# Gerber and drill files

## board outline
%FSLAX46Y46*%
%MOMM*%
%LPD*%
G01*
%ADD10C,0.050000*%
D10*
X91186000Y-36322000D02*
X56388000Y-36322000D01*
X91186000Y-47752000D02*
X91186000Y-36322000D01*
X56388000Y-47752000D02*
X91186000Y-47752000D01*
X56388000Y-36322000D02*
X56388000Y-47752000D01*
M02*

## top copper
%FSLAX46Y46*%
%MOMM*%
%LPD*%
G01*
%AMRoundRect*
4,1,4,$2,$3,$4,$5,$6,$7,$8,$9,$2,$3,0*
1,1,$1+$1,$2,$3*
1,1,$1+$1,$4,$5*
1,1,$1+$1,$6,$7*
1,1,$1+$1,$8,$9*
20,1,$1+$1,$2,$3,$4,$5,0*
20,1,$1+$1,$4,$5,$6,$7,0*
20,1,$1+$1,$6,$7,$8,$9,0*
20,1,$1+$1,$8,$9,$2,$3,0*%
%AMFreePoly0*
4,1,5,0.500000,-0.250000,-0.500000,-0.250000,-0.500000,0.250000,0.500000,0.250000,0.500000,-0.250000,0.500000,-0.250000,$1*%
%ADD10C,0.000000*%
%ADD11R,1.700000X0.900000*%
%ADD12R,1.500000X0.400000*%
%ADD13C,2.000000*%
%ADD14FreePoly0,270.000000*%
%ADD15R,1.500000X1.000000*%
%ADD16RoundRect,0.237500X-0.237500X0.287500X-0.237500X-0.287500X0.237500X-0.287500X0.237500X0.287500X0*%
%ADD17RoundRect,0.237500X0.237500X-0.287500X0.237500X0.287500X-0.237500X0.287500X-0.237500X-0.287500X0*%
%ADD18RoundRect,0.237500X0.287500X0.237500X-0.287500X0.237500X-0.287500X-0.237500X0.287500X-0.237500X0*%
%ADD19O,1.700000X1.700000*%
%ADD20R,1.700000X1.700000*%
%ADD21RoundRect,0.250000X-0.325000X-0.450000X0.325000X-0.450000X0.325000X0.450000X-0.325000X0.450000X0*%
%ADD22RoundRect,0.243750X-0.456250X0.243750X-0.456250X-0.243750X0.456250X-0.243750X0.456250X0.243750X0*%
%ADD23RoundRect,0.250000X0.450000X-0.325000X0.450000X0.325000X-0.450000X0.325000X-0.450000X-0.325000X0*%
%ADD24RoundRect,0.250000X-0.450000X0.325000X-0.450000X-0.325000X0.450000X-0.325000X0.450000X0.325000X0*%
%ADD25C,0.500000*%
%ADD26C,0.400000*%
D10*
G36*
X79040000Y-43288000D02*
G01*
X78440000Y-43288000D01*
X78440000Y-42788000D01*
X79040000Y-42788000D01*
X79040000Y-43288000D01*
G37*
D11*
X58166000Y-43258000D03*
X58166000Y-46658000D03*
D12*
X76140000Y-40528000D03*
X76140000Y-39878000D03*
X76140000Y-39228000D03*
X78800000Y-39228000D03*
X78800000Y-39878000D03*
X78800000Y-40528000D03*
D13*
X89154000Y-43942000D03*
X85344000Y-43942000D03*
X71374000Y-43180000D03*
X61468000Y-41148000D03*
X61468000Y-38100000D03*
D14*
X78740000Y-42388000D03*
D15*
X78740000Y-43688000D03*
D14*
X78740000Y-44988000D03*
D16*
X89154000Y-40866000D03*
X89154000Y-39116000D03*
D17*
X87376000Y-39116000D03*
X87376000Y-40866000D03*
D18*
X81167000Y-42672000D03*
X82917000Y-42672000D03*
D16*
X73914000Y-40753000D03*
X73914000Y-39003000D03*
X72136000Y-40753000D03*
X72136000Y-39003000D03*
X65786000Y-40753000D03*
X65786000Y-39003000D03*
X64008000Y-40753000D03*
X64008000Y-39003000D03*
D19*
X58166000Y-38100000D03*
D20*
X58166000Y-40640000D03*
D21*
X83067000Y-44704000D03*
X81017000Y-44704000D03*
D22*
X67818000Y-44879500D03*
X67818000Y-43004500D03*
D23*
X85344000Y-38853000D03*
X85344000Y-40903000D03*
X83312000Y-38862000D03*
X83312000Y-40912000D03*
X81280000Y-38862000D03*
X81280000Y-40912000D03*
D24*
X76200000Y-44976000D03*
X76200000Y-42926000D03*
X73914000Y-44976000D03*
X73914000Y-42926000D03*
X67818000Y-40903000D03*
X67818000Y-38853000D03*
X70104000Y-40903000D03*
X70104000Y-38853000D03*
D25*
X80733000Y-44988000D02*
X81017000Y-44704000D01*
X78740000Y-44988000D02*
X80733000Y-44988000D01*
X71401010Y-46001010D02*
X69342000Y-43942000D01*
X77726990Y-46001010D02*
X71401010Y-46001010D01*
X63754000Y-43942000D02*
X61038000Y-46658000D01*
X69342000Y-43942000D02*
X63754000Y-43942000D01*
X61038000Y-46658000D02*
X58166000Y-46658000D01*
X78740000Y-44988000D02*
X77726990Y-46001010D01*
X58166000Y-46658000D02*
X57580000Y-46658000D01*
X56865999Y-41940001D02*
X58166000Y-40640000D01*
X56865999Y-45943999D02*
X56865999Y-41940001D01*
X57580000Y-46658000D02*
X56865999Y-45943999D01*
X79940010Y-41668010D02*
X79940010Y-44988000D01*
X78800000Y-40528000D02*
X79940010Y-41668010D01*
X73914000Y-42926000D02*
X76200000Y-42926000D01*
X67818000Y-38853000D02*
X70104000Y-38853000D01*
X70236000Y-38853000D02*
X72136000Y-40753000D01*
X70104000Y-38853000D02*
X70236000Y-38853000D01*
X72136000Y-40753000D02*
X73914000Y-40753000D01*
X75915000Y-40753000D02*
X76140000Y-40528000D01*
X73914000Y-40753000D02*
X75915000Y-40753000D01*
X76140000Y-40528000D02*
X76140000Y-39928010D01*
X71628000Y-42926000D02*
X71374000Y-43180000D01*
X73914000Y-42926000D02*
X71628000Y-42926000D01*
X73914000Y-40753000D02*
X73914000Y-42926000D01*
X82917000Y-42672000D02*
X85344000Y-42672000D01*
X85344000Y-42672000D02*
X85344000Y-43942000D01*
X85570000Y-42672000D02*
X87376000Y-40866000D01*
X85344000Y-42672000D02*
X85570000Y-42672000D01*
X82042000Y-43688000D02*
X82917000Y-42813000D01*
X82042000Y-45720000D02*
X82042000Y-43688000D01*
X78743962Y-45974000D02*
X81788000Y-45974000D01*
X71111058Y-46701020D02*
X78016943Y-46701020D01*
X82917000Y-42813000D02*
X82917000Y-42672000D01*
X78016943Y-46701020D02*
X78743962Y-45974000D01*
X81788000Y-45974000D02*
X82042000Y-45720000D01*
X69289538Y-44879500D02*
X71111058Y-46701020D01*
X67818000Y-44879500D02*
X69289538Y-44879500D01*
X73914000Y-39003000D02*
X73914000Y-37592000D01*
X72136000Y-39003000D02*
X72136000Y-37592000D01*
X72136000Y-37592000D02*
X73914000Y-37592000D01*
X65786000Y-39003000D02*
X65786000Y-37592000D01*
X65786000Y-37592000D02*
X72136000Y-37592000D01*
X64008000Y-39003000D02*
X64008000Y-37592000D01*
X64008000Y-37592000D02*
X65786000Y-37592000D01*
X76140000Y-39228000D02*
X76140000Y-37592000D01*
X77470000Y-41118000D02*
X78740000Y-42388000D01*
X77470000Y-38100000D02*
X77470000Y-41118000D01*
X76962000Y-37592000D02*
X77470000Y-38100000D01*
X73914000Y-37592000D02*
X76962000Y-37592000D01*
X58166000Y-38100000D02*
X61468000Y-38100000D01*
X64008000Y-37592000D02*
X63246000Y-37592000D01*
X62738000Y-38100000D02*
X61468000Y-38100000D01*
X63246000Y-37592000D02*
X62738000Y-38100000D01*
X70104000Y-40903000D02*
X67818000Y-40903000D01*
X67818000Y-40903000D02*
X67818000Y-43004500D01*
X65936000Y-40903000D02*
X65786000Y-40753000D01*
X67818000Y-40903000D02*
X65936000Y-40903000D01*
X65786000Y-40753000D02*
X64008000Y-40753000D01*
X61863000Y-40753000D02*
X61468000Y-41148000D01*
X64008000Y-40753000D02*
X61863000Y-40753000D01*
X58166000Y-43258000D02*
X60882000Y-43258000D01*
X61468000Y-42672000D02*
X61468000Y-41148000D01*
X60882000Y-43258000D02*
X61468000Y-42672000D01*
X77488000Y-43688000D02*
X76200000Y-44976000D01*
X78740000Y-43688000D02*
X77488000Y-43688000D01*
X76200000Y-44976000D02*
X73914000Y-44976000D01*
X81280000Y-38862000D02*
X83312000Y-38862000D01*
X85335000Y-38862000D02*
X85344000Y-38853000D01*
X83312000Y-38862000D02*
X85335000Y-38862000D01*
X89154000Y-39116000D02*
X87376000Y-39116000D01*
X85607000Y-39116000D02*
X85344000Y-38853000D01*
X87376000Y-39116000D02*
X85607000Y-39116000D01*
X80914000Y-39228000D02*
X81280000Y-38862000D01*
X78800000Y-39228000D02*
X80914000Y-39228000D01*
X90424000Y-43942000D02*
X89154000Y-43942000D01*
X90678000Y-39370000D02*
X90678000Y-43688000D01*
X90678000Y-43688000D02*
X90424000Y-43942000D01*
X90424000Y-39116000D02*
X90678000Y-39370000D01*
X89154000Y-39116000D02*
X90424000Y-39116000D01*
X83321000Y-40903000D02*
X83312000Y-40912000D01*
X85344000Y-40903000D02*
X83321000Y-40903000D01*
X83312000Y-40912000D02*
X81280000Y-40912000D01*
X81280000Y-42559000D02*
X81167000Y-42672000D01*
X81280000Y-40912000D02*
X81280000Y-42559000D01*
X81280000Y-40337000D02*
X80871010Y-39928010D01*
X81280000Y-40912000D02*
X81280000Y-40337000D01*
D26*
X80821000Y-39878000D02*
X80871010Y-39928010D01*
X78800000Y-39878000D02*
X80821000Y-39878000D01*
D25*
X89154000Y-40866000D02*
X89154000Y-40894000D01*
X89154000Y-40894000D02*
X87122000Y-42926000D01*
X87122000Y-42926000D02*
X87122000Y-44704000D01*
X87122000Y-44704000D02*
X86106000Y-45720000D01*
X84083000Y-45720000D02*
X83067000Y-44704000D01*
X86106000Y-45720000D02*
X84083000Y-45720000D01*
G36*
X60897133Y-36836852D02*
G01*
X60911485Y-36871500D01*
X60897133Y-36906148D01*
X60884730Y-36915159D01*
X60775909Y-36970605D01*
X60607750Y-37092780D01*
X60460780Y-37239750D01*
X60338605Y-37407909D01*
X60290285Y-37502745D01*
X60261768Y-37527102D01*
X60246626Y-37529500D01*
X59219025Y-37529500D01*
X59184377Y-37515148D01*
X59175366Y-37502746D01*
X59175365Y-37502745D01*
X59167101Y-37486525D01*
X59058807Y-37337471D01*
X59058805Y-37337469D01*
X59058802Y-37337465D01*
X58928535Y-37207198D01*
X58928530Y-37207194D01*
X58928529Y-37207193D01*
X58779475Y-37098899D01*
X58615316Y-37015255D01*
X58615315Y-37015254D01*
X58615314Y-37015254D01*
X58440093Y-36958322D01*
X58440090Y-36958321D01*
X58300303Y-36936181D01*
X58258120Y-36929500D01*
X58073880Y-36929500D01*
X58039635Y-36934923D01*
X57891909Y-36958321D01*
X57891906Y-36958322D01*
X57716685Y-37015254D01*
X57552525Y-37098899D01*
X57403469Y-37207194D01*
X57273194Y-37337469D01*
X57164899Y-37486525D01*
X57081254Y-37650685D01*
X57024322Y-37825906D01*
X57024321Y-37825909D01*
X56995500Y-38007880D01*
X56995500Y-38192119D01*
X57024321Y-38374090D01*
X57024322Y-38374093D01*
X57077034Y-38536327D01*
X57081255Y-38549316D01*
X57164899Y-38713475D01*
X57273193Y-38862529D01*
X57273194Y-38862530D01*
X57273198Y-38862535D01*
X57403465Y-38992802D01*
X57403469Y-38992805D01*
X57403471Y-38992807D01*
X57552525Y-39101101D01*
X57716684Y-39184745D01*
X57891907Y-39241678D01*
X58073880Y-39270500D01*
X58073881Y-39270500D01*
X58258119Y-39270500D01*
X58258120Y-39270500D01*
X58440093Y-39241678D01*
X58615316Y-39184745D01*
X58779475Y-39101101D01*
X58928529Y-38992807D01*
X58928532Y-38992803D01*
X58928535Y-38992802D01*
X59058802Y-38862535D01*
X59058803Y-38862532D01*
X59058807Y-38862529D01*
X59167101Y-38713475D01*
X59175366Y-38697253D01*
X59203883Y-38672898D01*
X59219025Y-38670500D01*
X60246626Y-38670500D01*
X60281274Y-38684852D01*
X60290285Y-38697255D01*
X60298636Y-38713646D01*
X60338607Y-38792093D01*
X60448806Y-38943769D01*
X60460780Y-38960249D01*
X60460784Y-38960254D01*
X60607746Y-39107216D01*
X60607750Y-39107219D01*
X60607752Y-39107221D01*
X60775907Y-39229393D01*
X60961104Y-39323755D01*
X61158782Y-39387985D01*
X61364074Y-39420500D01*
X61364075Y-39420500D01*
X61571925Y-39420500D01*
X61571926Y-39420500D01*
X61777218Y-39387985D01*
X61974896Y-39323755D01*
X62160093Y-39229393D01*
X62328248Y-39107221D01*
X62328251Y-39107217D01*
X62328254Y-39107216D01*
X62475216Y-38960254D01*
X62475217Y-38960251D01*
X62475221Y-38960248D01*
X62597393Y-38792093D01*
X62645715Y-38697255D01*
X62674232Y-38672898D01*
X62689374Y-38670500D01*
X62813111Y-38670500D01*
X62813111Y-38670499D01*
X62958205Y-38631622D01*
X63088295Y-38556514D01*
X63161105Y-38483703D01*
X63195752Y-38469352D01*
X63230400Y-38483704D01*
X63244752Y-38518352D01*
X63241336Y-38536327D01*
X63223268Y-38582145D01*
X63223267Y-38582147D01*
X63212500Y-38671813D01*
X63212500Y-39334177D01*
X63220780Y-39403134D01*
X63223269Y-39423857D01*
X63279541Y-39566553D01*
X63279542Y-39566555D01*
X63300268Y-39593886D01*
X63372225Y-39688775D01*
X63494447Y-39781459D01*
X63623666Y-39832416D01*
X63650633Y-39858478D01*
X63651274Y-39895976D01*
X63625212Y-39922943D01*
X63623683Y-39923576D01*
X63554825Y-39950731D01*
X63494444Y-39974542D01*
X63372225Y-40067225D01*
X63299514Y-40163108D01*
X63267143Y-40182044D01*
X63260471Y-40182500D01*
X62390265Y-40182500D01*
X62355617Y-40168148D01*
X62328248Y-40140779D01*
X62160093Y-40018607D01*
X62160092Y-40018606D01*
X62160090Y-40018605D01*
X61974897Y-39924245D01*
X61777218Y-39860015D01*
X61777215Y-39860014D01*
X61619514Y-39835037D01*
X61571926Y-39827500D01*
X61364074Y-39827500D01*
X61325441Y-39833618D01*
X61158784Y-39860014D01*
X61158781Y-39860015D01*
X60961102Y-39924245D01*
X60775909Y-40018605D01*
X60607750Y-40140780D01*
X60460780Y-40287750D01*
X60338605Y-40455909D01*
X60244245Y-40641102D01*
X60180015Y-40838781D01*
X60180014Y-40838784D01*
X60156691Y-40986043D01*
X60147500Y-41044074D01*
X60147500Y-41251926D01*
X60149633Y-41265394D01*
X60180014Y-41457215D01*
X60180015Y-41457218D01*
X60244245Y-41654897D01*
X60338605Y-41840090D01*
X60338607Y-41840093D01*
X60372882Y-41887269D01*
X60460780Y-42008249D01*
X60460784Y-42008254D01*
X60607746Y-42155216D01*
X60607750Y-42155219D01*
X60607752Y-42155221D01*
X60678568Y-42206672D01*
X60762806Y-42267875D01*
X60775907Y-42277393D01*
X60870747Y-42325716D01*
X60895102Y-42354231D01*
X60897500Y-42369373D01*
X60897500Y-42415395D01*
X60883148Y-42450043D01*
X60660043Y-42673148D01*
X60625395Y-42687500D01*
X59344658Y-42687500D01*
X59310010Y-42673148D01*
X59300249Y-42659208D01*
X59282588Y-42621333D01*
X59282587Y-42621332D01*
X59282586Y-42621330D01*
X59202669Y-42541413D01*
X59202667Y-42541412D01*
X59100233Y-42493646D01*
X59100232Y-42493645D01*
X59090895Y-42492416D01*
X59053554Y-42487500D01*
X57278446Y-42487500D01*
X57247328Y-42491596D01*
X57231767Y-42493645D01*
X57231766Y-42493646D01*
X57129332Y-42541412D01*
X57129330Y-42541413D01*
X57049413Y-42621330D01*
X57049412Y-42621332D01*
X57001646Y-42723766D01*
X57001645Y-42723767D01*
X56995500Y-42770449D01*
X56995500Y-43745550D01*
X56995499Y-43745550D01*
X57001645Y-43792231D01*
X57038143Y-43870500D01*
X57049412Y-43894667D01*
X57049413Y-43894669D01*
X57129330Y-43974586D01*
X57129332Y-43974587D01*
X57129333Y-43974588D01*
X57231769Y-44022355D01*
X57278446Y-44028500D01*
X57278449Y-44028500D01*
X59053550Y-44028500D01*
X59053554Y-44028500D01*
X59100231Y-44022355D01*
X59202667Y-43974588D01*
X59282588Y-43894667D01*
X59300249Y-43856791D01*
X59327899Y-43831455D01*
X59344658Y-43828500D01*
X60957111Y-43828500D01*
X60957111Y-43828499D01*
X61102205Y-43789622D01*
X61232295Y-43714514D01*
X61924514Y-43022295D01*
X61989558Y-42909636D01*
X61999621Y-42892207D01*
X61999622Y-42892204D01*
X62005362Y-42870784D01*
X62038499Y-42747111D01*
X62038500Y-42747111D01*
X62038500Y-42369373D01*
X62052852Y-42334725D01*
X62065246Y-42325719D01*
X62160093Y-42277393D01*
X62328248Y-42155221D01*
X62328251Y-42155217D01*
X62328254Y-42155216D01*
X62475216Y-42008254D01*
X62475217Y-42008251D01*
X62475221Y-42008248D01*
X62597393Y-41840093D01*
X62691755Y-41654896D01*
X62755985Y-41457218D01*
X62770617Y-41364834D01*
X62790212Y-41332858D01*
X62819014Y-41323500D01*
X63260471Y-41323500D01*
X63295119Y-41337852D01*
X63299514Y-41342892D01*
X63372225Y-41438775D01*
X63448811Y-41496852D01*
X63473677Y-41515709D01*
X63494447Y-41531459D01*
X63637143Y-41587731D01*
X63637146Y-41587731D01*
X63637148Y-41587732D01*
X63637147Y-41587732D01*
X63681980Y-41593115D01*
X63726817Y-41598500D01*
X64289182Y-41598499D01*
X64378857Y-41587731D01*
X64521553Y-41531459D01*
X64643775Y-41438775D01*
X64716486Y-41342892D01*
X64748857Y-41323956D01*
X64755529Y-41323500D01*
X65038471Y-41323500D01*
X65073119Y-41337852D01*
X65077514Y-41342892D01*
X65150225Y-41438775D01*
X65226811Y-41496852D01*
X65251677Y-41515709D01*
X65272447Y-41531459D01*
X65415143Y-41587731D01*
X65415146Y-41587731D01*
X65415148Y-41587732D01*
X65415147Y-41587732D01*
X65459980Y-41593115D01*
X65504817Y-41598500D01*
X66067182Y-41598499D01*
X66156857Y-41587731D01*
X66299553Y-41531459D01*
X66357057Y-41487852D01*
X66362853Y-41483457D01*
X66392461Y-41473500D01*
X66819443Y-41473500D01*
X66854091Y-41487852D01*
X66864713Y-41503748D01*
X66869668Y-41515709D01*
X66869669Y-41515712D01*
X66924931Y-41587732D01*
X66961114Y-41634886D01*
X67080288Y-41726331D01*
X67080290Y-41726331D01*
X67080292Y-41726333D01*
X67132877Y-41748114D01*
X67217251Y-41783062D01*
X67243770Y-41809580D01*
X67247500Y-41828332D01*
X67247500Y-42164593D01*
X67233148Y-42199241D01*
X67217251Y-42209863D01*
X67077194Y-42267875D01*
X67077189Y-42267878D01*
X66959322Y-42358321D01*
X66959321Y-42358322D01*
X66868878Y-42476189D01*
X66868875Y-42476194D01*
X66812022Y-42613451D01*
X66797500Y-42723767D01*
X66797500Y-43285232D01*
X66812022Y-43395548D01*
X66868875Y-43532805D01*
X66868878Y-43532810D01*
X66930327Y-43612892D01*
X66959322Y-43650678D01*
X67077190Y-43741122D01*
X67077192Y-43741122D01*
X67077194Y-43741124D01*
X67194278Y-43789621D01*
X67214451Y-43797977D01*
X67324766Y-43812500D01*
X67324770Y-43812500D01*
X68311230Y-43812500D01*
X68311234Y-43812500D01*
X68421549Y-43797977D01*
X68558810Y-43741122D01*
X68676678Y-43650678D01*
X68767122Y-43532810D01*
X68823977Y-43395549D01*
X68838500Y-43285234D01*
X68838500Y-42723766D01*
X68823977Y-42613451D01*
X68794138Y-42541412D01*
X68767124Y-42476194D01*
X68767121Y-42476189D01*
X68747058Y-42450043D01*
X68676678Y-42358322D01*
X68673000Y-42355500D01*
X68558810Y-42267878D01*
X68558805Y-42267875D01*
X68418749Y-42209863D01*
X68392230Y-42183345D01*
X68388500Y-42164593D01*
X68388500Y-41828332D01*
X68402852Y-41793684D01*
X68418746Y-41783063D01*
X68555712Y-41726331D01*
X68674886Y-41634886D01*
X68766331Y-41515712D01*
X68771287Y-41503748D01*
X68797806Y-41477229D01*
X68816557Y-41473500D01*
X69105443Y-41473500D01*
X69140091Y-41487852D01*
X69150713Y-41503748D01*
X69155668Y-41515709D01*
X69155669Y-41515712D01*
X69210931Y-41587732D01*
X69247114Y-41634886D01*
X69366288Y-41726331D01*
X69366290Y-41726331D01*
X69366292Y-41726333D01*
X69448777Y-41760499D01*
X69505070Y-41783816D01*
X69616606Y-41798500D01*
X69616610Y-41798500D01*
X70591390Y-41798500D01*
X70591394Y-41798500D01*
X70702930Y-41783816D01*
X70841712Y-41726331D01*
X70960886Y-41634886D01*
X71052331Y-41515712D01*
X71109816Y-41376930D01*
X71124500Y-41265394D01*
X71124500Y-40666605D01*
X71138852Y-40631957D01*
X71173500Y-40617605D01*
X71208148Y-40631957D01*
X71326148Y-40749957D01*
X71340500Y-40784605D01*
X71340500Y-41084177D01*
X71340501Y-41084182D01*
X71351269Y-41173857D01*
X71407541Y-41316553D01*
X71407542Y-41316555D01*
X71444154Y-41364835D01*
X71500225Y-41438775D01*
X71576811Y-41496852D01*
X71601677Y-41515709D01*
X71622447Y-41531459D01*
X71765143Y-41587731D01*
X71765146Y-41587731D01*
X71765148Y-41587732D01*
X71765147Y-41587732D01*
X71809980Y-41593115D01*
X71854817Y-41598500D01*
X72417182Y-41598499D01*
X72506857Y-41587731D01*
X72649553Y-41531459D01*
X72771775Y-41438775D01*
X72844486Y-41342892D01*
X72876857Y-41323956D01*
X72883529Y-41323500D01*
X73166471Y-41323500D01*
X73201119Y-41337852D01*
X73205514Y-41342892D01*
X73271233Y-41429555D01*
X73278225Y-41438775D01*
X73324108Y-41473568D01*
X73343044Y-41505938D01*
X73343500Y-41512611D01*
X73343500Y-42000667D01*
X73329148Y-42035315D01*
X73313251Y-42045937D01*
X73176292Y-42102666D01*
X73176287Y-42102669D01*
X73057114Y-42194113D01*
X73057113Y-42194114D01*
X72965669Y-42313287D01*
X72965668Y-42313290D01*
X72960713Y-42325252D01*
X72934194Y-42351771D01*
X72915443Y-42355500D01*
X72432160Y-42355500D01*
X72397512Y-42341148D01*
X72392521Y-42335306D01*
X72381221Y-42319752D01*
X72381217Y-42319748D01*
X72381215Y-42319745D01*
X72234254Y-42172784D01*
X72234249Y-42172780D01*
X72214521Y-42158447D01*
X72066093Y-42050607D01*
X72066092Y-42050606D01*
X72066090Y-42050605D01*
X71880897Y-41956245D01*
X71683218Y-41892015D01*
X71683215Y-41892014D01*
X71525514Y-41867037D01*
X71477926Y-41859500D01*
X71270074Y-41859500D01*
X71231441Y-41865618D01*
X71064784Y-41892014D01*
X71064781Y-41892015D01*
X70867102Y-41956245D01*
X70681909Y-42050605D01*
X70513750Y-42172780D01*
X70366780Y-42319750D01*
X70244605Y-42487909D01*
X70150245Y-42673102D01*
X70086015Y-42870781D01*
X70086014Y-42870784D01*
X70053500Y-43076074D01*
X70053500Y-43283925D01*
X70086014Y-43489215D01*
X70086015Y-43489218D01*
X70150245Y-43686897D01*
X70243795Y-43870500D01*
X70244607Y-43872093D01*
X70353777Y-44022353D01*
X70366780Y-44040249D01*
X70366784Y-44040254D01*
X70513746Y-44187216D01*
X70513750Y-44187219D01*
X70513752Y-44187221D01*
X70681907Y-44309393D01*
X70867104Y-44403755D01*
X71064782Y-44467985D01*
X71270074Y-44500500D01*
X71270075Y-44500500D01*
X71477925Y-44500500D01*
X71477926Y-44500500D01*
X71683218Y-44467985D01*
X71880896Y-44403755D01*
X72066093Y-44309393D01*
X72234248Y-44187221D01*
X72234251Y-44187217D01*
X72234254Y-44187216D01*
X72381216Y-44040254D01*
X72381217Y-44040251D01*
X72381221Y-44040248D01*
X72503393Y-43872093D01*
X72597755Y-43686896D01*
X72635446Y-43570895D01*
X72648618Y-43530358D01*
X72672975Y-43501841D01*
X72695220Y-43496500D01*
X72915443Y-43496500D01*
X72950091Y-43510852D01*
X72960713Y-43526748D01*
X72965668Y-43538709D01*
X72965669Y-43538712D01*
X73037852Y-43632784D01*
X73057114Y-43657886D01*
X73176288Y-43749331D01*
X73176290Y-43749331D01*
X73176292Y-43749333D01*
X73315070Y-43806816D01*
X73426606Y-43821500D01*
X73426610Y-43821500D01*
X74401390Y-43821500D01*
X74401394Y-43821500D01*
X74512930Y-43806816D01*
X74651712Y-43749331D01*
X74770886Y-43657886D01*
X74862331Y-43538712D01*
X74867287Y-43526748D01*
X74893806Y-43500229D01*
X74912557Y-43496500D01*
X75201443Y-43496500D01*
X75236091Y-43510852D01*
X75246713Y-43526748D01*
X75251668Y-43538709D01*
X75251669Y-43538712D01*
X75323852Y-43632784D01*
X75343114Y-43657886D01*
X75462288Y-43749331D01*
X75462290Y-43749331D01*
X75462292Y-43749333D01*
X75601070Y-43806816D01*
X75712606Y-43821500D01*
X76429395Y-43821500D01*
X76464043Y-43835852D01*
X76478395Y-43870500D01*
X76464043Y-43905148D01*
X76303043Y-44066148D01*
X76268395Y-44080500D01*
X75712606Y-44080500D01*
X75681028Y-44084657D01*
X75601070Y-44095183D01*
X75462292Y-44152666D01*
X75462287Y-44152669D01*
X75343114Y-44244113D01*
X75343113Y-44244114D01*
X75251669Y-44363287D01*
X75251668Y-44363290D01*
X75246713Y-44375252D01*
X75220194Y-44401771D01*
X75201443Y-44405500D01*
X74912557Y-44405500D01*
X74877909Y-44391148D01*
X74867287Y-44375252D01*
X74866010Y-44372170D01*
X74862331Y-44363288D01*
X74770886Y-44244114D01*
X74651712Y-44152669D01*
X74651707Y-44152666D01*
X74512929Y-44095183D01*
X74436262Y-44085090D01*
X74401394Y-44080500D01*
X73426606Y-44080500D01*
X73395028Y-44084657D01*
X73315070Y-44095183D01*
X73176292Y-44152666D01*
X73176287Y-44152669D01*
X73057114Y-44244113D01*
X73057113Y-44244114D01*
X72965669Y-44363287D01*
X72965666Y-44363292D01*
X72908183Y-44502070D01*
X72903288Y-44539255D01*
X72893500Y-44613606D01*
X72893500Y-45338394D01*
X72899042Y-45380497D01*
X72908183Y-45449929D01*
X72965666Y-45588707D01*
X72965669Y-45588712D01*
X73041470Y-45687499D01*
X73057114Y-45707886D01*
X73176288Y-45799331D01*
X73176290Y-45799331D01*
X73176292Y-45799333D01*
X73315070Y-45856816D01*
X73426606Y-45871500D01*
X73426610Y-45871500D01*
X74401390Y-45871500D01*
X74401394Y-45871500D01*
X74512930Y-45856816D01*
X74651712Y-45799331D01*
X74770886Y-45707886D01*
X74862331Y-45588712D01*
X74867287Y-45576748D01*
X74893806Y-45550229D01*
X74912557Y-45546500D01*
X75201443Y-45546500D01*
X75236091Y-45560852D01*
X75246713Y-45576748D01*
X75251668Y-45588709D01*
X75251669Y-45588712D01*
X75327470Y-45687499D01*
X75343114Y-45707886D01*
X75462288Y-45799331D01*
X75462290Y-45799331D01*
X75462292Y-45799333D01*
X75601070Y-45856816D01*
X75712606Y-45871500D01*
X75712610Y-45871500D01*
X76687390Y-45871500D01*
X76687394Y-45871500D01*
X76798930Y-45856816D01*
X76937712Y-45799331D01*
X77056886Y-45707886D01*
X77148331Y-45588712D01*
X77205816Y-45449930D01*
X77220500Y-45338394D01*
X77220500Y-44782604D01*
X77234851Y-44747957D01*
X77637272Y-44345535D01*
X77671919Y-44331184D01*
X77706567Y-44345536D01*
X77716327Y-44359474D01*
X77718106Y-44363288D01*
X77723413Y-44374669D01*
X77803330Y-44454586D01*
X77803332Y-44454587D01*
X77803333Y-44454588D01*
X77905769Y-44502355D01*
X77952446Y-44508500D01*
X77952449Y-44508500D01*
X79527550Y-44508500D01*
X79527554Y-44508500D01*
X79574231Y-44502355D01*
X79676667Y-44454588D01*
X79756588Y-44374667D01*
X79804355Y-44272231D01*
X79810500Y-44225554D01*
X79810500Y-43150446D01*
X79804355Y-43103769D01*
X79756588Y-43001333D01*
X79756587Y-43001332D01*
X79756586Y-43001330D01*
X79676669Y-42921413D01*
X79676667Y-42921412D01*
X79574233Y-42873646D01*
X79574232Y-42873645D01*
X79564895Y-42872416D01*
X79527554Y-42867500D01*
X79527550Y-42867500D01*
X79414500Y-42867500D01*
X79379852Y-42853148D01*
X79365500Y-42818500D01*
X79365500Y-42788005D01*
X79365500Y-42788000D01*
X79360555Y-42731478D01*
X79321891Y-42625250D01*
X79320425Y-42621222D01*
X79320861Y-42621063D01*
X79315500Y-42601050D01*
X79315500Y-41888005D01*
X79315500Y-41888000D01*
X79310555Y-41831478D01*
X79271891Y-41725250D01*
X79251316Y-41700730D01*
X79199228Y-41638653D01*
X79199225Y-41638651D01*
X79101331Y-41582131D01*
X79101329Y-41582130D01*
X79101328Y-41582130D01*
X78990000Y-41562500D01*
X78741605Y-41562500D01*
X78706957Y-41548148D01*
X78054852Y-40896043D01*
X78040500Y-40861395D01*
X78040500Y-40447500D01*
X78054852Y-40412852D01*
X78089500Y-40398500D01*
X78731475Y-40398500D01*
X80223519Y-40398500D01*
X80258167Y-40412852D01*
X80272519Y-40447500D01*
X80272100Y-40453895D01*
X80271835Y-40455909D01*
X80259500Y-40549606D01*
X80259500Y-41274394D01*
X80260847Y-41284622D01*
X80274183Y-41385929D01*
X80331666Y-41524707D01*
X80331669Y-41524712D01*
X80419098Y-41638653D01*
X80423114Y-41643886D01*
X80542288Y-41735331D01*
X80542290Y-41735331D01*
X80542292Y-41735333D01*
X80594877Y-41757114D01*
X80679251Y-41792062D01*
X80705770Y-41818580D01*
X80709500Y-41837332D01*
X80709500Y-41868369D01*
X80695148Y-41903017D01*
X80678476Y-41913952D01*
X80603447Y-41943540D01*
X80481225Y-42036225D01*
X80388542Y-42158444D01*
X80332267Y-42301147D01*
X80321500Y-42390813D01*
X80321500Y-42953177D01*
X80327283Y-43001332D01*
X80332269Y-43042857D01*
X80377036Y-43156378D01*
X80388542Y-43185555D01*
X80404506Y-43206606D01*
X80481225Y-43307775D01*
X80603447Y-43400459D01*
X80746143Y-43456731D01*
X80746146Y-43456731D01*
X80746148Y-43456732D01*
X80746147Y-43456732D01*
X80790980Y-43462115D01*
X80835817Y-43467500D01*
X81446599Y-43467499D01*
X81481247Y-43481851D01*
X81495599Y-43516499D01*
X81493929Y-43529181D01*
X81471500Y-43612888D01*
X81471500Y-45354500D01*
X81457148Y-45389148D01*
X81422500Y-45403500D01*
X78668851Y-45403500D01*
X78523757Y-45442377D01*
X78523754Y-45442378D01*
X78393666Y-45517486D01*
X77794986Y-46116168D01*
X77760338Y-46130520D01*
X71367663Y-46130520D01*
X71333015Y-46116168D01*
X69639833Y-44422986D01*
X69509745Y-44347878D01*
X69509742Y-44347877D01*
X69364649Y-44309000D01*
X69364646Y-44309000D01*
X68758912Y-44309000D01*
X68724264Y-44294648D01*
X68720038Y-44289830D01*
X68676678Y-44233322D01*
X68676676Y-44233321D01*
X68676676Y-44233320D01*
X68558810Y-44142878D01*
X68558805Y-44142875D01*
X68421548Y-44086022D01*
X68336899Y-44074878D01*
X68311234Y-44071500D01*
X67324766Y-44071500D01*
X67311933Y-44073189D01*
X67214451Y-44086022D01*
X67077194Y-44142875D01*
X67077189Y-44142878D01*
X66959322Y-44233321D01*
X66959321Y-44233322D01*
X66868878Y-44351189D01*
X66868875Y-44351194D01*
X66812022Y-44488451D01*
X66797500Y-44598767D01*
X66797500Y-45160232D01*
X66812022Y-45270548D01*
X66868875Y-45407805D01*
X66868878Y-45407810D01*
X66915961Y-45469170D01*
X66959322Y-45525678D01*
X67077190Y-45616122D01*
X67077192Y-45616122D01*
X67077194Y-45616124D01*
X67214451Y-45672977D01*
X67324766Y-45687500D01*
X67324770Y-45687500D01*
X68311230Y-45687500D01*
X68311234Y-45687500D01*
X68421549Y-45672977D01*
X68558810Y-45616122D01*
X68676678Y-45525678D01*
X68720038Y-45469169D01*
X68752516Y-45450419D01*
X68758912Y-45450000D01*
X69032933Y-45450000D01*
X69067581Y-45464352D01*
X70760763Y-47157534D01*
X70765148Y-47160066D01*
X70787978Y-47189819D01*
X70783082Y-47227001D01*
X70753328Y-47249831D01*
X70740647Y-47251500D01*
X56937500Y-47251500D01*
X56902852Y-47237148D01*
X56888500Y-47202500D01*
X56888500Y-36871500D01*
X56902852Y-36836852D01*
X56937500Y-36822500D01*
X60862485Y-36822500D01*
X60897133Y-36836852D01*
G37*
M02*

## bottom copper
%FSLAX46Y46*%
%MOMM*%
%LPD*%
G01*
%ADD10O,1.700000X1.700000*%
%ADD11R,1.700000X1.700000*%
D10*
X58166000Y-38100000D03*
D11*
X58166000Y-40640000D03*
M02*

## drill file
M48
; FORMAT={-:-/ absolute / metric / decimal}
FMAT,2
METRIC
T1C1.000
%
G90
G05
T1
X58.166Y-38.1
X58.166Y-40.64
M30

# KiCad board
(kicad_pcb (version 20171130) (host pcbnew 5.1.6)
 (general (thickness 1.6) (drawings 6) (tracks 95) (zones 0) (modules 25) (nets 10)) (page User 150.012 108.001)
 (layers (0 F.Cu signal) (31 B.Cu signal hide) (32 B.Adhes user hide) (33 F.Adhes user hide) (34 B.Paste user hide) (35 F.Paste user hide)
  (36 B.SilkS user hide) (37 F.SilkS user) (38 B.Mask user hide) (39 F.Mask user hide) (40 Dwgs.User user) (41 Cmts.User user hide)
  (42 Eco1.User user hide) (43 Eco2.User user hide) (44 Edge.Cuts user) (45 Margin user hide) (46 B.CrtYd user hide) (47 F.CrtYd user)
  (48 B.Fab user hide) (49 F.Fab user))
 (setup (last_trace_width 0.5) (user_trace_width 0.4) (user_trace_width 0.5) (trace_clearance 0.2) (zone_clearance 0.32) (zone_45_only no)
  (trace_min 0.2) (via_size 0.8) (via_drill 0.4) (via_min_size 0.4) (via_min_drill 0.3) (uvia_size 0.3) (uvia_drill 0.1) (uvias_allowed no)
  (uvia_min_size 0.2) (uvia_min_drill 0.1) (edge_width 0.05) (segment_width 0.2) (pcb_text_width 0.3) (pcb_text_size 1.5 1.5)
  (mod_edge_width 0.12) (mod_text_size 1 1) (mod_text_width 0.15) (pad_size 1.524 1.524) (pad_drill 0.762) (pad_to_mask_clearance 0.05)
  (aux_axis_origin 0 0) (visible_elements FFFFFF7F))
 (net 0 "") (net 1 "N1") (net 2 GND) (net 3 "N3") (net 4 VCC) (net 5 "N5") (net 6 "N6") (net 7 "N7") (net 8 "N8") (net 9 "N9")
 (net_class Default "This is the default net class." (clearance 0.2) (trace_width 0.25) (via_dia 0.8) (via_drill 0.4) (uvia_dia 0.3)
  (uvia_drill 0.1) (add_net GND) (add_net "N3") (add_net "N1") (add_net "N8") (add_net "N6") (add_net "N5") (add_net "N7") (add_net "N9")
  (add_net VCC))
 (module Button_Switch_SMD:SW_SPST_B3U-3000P (layer F.Cu) (at 58.166 44.958 90)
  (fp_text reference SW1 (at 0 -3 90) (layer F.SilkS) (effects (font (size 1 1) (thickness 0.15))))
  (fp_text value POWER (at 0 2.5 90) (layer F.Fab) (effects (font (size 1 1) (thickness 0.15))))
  (pad 2 smd rect (at 1.7 0 90) (size 0.9 1.7) (layers F.Cu F.Paste F.Mask) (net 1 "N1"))
  (pad 1 smd rect (at -1.7 0 90) (size 0.9 1.7) (layers F.Cu F.Paste F.Mask) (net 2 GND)))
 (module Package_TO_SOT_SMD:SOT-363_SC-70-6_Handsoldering (layer F.Cu) (at 77.47 39.878 180)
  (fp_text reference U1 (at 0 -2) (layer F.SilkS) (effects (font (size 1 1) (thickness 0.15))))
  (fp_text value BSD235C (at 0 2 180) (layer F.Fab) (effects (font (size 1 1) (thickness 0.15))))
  (pad 6 smd rect (at 1.33 -0.65 180) (size 1.5 0.4) (layers F.Cu F.Paste F.Mask) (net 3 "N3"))
  (pad 5 smd rect (at 1.33 0 180) (size 1.5 0.4) (layers F.Cu F.Paste F.Mask) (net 3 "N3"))
  (pad 4 smd rect (at 1.33 0.65 180) (size 1.5 0.4) (layers F.Cu F.Paste F.Mask) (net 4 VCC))
  (pad 3 smd rect (at -1.33 0.65 180) (size 1.5 0.4) (layers F.Cu F.Paste F.Mask) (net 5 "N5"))
  (pad 2 smd rect (at -1.33 0 180) (size 1.5 0.4) (layers F.Cu F.Paste F.Mask) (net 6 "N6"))
  (pad 1 smd rect (at -1.33 -0.65 180) (size 1.5 0.4) (layers F.Cu F.Paste F.Mask) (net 2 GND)))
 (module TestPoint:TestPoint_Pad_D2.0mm (layer F.Cu) (at 89.154 43.942)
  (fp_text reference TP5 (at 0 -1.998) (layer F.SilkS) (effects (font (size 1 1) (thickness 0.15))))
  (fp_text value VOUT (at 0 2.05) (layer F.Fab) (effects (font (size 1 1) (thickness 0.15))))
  (pad 1 smd circle (at 0 0) (size 2 2) (layers F.Cu F.Mask) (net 5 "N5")))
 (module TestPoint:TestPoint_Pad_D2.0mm (layer F.Cu) (at 85.344 43.942)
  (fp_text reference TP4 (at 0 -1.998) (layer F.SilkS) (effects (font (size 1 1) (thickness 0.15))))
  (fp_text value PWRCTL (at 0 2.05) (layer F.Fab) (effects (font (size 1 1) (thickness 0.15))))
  (pad 1 smd circle (at 0 0) (size 2 2) (layers F.Cu F.Mask) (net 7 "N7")))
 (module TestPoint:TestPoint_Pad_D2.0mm (layer F.Cu) (at 71.374 43.18)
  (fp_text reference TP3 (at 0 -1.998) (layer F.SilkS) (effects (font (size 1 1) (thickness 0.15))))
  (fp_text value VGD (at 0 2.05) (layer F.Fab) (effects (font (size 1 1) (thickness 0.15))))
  (pad 1 smd circle (at 0 0) (size 2 2) (layers F.Cu F.Mask) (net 3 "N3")))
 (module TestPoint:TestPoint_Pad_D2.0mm (layer F.Cu) (at 61.468 41.148)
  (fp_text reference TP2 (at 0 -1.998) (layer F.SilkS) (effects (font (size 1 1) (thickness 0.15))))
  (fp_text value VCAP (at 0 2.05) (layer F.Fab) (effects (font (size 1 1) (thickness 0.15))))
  (pad 1 smd circle (at 0 0) (size 2 2) (layers F.Cu F.Mask) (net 1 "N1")))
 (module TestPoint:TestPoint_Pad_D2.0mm (layer F.Cu) (at 61.468 38.1)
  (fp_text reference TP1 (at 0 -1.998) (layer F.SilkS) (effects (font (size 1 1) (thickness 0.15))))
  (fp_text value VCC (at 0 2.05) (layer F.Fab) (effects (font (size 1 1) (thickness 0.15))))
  (pad 1 smd circle (at 0 0) (size 2 2) (layers F.Cu F.Mask) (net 4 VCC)))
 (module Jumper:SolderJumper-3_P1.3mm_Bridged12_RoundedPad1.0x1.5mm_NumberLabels (layer F.Cu) (at 78.74 43.688 270)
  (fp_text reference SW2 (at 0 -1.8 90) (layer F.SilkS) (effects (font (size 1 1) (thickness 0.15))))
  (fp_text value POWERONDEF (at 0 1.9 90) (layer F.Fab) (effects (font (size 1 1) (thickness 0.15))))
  (fp_poly (pts (xy -0.9 -0.3) (xy -0.4 -0.3) (xy -0.4 0.3) (xy -0.9 0.3)) (layer F.Cu) (width 0))
  (pad 1 smd custom (at -1.3 0 270) (size 1 0.5) (layers F.Cu F.Mask) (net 4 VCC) (zone_connect 2)
   (options (clearance outline) (anchor rect)) (primitives))
  (pad 2 smd rect (at 0 0 270) (size 1 1.5) (layers F.Cu F.Mask) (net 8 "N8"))
  (pad 3 smd custom (at 1.3 0 270) (size 1 0.5) (layers F.Cu F.Mask) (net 2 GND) (zone_connect 2)
   (options (clearance outline) (anchor rect)) (primitives)))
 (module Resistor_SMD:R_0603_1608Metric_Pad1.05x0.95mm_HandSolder (layer F.Cu) (at 89.154 39.991 270)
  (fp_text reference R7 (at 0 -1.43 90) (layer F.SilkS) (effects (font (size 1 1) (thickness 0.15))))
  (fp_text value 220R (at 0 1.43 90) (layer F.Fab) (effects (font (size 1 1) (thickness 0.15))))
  (pad 2 smd roundrect (at 0.875 0 270) (size 1.05 0.95) (layers F.Cu F.Paste F.Mask) (roundrect_rratio 0.25) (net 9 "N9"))
  (pad 1 smd roundrect (at -0.875 0 270) (size 1.05 0.95) (layers F.Cu F.Paste F.Mask) (roundrect_rratio 0.25) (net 5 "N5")))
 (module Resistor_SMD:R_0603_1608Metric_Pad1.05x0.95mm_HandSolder (layer F.Cu) (at 87.376 39.991 90)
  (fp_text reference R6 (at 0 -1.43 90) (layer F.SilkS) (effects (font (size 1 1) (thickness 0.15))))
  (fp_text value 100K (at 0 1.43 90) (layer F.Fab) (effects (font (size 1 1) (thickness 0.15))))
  (pad 2 smd roundrect (at 0.875 0 90) (size 1.05 0.95) (layers F.Cu F.Paste F.Mask) (roundrect_rratio 0.25) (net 5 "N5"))
  (pad 1 smd roundrect (at -0.875 0 90) (size 1.05 0.95) (layers F.Cu F.Paste F.Mask) (roundrect_rratio 0.25) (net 7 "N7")))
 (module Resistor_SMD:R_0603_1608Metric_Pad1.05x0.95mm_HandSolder (layer F.Cu) (at 82.042 42.672 180)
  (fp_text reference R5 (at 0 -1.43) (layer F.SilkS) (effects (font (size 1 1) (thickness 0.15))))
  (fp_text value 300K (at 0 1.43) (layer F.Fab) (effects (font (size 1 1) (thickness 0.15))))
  (pad 2 smd roundrect (at 0.875 0 180) (size 1.05 0.95) (layers F.Cu F.Paste F.Mask) (roundrect_rratio 0.25) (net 6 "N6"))
  (pad 1 smd roundrect (at -0.875 0 180) (size 1.05 0.95) (layers F.Cu F.Paste F.Mask) (roundrect_rratio 0.25) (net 7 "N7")))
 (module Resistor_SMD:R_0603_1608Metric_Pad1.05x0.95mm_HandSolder (layer F.Cu) (at 73.914 39.878 270)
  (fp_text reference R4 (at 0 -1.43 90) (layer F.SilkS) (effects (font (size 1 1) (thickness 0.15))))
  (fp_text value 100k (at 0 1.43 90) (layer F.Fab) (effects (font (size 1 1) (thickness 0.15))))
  (pad 2 smd roundrect (at 0.875 0 270) (size 1.05 0.95) (layers F.Cu F.Paste F.Mask) (roundrect_rratio 0.25) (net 3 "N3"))
  (pad 1 smd roundrect (at -0.875 0 270) (size 1.05 0.95) (layers F.Cu F.Paste F.Mask) (roundrect_rratio 0.25) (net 4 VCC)))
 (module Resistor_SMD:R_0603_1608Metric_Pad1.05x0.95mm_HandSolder (layer F.Cu) (at 72.136 39.878 270)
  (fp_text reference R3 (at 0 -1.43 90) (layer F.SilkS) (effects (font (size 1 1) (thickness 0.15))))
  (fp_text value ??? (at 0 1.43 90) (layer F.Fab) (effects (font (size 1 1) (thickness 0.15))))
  (pad 2 smd roundrect (at 0.875 0 270) (size 1.05 0.95) (layers F.Cu F.Paste F.Mask) (roundrect_rratio 0.25) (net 3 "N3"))
  (pad 1 smd roundrect (at -0.875 0 270) (size 1.05 0.95) (layers F.Cu F.Paste F.Mask) (roundrect_rratio 0.25) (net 4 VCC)))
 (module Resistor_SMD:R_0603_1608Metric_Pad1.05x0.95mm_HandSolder (layer F.Cu) (at 65.786 39.878 270)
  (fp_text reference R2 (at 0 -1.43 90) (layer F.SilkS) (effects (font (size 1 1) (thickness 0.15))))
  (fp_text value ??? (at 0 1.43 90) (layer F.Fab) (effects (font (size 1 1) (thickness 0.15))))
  (pad 2 smd roundrect (at 0.875 0 270) (size 1.05 0.95) (layers F.Cu F.Paste F.Mask) (roundrect_rratio 0.25) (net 1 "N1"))
  (pad 1 smd roundrect (at -0.875 0 270) (size 1.05 0.95) (layers F.Cu F.Paste F.Mask) (roundrect_rratio 0.25) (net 4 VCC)))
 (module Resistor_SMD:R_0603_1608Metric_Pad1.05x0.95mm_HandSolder (layer F.Cu) (at 64.008 39.878 270)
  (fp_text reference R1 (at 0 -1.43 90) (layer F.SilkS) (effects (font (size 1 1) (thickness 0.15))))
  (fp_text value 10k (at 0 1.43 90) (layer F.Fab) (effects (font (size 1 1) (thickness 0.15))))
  (pad 2 smd roundrect (at 0.875 0 270) (size 1.05 0.95) (layers F.Cu F.Paste F.Mask) (roundrect_rratio 0.25) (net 1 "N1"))
  (pad 1 smd roundrect (at -0.875 0 270) (size 1.05 0.95) (layers F.Cu F.Paste F.Mask) (roundrect_rratio 0.25) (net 4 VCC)))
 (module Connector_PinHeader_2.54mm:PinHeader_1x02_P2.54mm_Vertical (layer F.Cu) (at 58.166 40.64 180)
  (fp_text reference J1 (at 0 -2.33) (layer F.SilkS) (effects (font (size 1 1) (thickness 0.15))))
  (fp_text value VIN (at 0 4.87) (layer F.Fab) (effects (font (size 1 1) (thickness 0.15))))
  (pad 2 thru_hole oval (at 0 2.54 180) (size 1.7 1.7) (drill 1) (layers *.Cu *.Mask) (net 4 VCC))
  (pad 1 thru_hole rect (at 0 0 180) (size 1.7 1.7) (drill 1) (layers *.Cu *.Mask) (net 2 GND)))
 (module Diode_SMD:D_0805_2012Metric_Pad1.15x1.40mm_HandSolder (layer F.Cu) (at 82.042 44.704)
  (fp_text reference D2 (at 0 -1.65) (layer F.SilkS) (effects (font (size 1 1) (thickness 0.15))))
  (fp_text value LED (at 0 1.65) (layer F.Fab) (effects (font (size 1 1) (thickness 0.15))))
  (pad 2 smd roundrect (at 1.025 0) (size 1.15 1.4) (layers F.Cu F.Paste F.Mask) (roundrect_rratio 0.217391) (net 9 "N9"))
  (pad 1 smd roundrect (at -1.025 0) (size 1.15 1.4) (layers F.Cu F.Paste F.Mask) (roundrect_rratio 0.217391) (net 2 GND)))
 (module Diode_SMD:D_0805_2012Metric (layer F.Cu) (at 67.818 43.942 270)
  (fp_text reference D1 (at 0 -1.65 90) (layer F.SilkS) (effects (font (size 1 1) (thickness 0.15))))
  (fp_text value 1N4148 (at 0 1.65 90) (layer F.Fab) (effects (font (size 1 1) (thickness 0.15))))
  (pad 2 smd roundrect (at 0.9375 0 270) (size 0.975 1.4) (layers F.Cu F.Paste F.Mask) (roundrect_rratio 0.25) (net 7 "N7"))
  (pad 1 smd roundrect (at -0.9375 0 270) (size 0.975 1.4) (layers F.Cu F.Paste F.Mask) (roundrect_rratio 0.25) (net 1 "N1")))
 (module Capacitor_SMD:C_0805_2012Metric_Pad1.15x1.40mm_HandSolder (layer F.Cu) (at 85.344 39.878 90)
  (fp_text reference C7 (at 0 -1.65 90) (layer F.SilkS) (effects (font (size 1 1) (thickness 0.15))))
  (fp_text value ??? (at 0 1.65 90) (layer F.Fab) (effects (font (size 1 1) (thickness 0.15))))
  (pad 2 smd roundrect (at 1.025 0 90) (size 1.15 1.4) (layers F.Cu F.Paste F.Mask) (roundrect_rratio 0.217391) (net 5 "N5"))
  (pad 1 smd roundrect (at -1.025 0 90) (size 1.15 1.4) (layers F.Cu F.Paste F.Mask) (roundrect_rratio 0.217391) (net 6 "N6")))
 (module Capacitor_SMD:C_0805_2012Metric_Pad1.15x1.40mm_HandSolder (layer F.Cu) (at 83.312 39.887 90)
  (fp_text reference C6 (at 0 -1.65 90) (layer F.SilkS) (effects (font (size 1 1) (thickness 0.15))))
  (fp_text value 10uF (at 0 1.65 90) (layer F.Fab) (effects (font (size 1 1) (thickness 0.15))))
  (pad 2 smd roundrect (at 1.025 0 90) (size 1.15 1.4) (layers F.Cu F.Paste F.Mask) (roundrect_rratio 0.217391) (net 5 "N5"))
  (pad 1 smd roundrect (at -1.025 0 90) (size 1.15 1.4) (layers F.Cu F.Paste F.Mask) (roundrect_rratio 0.217391) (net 6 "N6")))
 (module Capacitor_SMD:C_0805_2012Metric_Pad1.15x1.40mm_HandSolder (layer F.Cu) (at 81.28 39.887 90)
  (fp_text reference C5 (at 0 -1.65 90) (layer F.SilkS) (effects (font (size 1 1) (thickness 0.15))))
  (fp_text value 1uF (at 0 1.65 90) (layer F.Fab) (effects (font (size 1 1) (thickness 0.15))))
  (pad 2 smd roundrect (at 1.025 0 90) (size 1.15 1.4) (layers F.Cu F.Paste F.Mask) (roundrect_rratio 0.217391) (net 5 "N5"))
  (pad 1 smd roundrect (at -1.025 0 90) (size 1.15 1.4) (layers F.Cu F.Paste F.Mask) (roundrect_rratio 0.217391) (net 6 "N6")))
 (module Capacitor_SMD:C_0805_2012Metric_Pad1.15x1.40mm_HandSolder (layer F.Cu) (at 76.2 43.951 270)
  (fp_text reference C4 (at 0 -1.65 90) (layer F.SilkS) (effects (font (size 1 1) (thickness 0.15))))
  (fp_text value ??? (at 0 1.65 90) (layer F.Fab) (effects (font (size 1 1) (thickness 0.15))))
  (pad 2 smd roundrect (at 1.025 0 270) (size 1.15 1.4) (layers F.Cu F.Paste F.Mask) (roundrect_rratio 0.217391) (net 8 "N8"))
  (pad 1 smd roundrect (at -1.025 0 270) (size 1.15 1.4) (layers F.Cu F.Paste F.Mask) (roundrect_rratio 0.217391) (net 3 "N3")))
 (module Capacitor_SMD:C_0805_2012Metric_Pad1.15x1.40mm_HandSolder (layer F.Cu) (at 73.914 43.951 270)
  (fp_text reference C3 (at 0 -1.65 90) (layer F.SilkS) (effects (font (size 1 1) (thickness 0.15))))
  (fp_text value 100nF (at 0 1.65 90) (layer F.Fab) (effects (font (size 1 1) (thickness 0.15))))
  (pad 2 smd roundrect (at 1.025 0 270) (size 1.15 1.4) (layers F.Cu F.Paste F.Mask) (roundrect_rratio 0.217391) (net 8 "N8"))
  (pad 1 smd roundrect (at -1.025 0 270) (size 1.15 1.4) (layers F.Cu F.Paste F.Mask) (roundrect_rratio 0.217391) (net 3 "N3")))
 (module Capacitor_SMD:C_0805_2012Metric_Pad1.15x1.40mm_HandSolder (layer F.Cu) (at 67.818 39.878 270)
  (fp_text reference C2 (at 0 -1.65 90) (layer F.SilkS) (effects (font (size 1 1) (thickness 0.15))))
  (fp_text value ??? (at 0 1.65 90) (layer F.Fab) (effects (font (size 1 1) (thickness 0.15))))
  (pad 2 smd roundrect (at 1.025 0 270) (size 1.15 1.4) (layers F.Cu F.Paste F.Mask) (roundrect_rratio 0.217391) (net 1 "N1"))
  (pad 1 smd roundrect (at -1.025 0 270) (size 1.15 1.4) (layers F.Cu F.Paste F.Mask) (roundrect_rratio 0.217391) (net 3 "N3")))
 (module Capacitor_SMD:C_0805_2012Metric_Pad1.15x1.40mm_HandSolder (layer F.Cu) (at 70.104 39.878 270)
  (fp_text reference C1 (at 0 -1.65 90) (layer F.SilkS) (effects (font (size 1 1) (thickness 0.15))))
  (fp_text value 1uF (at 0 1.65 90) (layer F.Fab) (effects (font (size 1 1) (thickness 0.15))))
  (pad 2 smd roundrect (at 1.025 0 270) (size 1.15 1.4) (layers F.Cu F.Paste F.Mask) (roundrect_rratio 0.217391) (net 1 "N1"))
  (pad 1 smd roundrect (at -1.025 0 270) (size 1.15 1.4) (layers F.Cu F.Paste F.Mask) (roundrect_rratio 0.217391) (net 3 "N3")))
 (gr_line (start 91.186 36.322) (end 56.388 36.322) (layer Edge.Cuts) (width 0.05))
 (gr_line (start 91.186 47.752) (end 91.186 36.322) (layer Edge.Cuts) (width 0.05))
 (gr_line (start 56.388 47.752) (end 91.186 47.752) (layer Edge.Cuts) (width 0.05))
 (gr_line (start 56.388 36.322) (end 56.388 47.752) (layer Edge.Cuts) (width 0.05))
 (segment (start 80.733 44.988) (end 81.017 44.704) (width 0.5) (layer F.Cu) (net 2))
 (segment (start 78.74 44.988) (end 80.733 44.988) (width 0.5) (layer F.Cu) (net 2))
 (segment (start 71.40101 46.00101) (end 69.342 43.942) (width 0.5) (layer F.Cu) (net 2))
 (segment (start 77.72699 46.00101) (end 71.40101 46.00101) (width 0.5) (layer F.Cu) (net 2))
 (segment (start 63.754 43.942) (end 61.038 46.658) (width 0.5) (layer F.Cu) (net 2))
 (segment (start 69.342 43.942) (end 63.754 43.942) (width 0.5) (layer F.Cu) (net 2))
 (segment (start 61.038 46.658) (end 58.166 46.658) (width 0.5) (layer F.Cu) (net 2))
 (segment (start 78.74 44.988) (end 77.72699 46.00101) (width 0.5) (layer F.Cu) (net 2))
 (segment (start 58.166 46.658) (end 57.58 46.658) (width 0.5) (layer F.Cu) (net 2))
 (segment (start 56.865999 41.940001) (end 58.166 40.64) (width 0.5) (layer F.Cu) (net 2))
 (segment (start 56.865999 45.943999) (end 56.865999 41.940001) (width 0.5) (layer F.Cu) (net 2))
 (segment (start 57.58 46.658) (end 56.865999 45.943999) (width 0.5) (layer F.Cu) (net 2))
 (segment (start 79.94001 41.66801) (end 79.94001 44.988) (width 0.5) (layer F.Cu) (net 2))
 (segment (start 78.8 40.528) (end 79.94001 41.66801) (width 0.5) (layer F.Cu) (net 2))
 (segment (start 73.914 42.926) (end 76.2 42.926) (width 0.5) (layer F.Cu) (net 3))
 (segment (start 67.818 38.853) (end 70.104 38.853) (width 0.5) (layer F.Cu) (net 3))
 (segment (start 70.236 38.853) (end 72.136 40.753) (width 0.5) (layer F.Cu) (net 3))
 (segment (start 70.104 38.853) (end 70.236 38.853) (width 0.5) (layer F.Cu) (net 3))
 (segment (start 72.136 40.753) (end 73.914 40.753) (width 0.5) (layer F.Cu) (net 3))
 (segment (start 75.915 40.753) (end 76.14 40.528) (width 0.5) (layer F.Cu) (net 3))
 (segment (start 73.914 40.753) (end 75.915 40.753) (width 0.5) (layer F.Cu) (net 3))
 (segment (start 76.14 40.528) (end 76.14 39.92801) (width 0.5) (layer F.Cu) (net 3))
 (segment (start 71.628 42.926) (end 71.374 43.18) (width 0.5) (layer F.Cu) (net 3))
 (segment (start 73.914 42.926) (end 71.628 42.926) (width 0.5) (layer F.Cu) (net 3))
 (segment (start 73.914 40.753) (end 73.914 42.926) (width 0.5) (layer F.Cu) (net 3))
 (segment (start 82.917 42.672) (end 85.344 42.672) (width 0.5) (layer F.Cu) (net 7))
 (segment (start 85.344 42.672) (end 85.344 43.942) (width 0.5) (layer F.Cu) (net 7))
 (segment (start 85.57 42.672) (end 87.376 40.866) (width 0.5) (layer F.Cu) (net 7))
 (segment (start 85.344 42.672) (end 85.57 42.672) (width 0.5) (layer F.Cu) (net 7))
 (segment (start 82.042 43.688) (end 82.917 42.813) (width 0.5) (layer F.Cu) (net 7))
 (segment (start 82.042 45.72) (end 82.042 43.688) (width 0.5) (layer F.Cu) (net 7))
 (segment (start 78.743962 45.974) (end 81.788 45.974) (width 0.5) (layer F.Cu) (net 7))
 (segment (start 71.111058 46.70102) (end 78.016943 46.70102) (width 0.5) (layer F.Cu) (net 7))
 (segment (start 82.917 42.813) (end 82.917 42.672) (width 0.5) (layer F.Cu) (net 7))
 (segment (start 78.016943 46.70102) (end 78.743962 45.974) (width 0.5) (layer F.Cu) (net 7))
 (segment (start 81.788 45.974) (end 82.042 45.72) (width 0.5) (layer F.Cu) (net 7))
 (segment (start 69.289538 44.8795) (end 71.111058 46.70102) (width 0.5) (layer F.Cu) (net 7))
 (segment (start 67.818 44.8795) (end 69.289538 44.8795) (width 0.5) (layer F.Cu) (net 7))
 (segment (start 73.914 39.003) (end 73.914 37.592) (width 0.5) (layer F.Cu) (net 4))
 (segment (start 72.136 39.003) (end 72.136 37.592) (width 0.5) (layer F.Cu) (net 4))
 (segment (start 72.136 37.592) (end 73.914 37.592) (width 0.5) (layer F.Cu) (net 4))
 (segment (start 65.786 39.003) (end 65.786 37.592) (width 0.5) (layer F.Cu) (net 4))
 (segment (start 65.786 37.592) (end 72.136 37.592) (width 0.5) (layer F.Cu) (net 4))
 (segment (start 64.008 39.003) (end 64.008 37.592) (width 0.5) (layer F.Cu) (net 4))
 (segment (start 64.008 37.592) (end 65.786 37.592) (width 0.5) (layer F.Cu) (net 4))
 (segment (start 76.14 39.228) (end 76.14 37.592) (width 0.5) (layer F.Cu) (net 4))
 (segment (start 77.47 41.118) (end 78.74 42.388) (width 0.5) (layer F.Cu) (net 4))
 (segment (start 77.47 38.1) (end 77.47 41.118) (width 0.5) (layer F.Cu) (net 4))
 (segment (start 76.962 37.592) (end 77.47 38.1) (width 0.5) (layer F.Cu) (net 4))
 (segment (start 73.914 37.592) (end 76.962 37.592) (width 0.5) (layer F.Cu) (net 4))
 (segment (start 58.166 38.1) (end 61.468 38.1) (width 0.5) (layer F.Cu) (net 4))
 (segment (start 64.008 37.592) (end 63.246 37.592) (width 0.5) (layer F.Cu) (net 4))
 (segment (start 62.738 38.1) (end 61.468 38.1) (width 0.5) (layer F.Cu) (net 4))
 (segment (start 63.246 37.592) (end 62.738 38.1) (width 0.5) (layer F.Cu) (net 4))
 (segment (start 70.104 40.903) (end 67.818 40.903) (width 0.5) (layer F.Cu) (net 1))
 (segment (start 67.818 40.903) (end 67.818 43.0045) (width 0.5) (layer F.Cu) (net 1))
 (segment (start 65.936 40.903) (end 65.786 40.753) (width 0.5) (layer F.Cu) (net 1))
 (segment (start 67.818 40.903) (end 65.936 40.903) (width 0.5) (layer F.Cu) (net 1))
 (segment (start 65.786 40.753) (end 64.008 40.753) (width 0.5) (layer F.Cu) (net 1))
 (segment (start 61.863 40.753) (end 61.468 41.148) (width 0.5) (layer F.Cu) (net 1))
 (segment (start 64.008 40.753) (end 61.863 40.753) (width 0.5) (layer F.Cu) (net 1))
 (segment (start 58.166 43.258) (end 60.882 43.258) (width 0.5) (layer F.Cu) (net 1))
 (segment (start 61.468 42.672) (end 61.468 41.148) (width 0.5) (layer F.Cu) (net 1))
 (segment (start 60.882 43.258) (end 61.468 42.672) (width 0.5) (layer F.Cu) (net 1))
 (segment (start 77.488 43.688) (end 76.2 44.976) (width 0.5) (layer F.Cu) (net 8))
 (segment (start 78.74 43.688) (end 77.488 43.688) (width 0.5) (layer F.Cu) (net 8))
 (segment (start 76.2 44.976) (end 73.914 44.976) (width 0.5) (layer F.Cu) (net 8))
 (segment (start 81.28 38.862) (end 83.312 38.862) (width 0.5) (layer F.Cu) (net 5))
 (segment (start 85.335 38.862) (end 85.344 38.853) (width 0.5) (layer F.Cu) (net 5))
 (segment (start 83.312 38.862) (end 85.335 38.862) (width 0.5) (layer F.Cu) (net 5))
 (segment (start 89.154 39.116) (end 87.376 39.116) (width 0.5) (layer F.Cu) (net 5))
 (segment (start 85.607 39.116) (end 85.344 38.853) (width 0.5) (layer F.Cu) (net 5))
 (segment (start 87.376 39.116) (end 85.607 39.116) (width 0.5) (layer F.Cu) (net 5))
 (segment (start 80.914 39.228) (end 81.28 38.862) (width 0.5) (layer F.Cu) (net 5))
 (segment (start 78.8 39.228) (end 80.914 39.228) (width 0.5) (layer F.Cu) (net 5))
 (segment (start 90.424 43.942) (end 89.154 43.942) (width 0.5) (layer F.Cu) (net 5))
 (segment (start 90.678 39.37) (end 90.678 43.688) (width 0.5) (layer F.Cu) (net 5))
 (segment (start 90.678 43.688) (end 90.424 43.942) (width 0.5) (layer F.Cu) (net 5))
 (segment (start 90.424 39.116) (end 90.678 39.37) (width 0.5) (layer F.Cu) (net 5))
 (segment (start 89.154 39.116) (end 90.424 39.116) (width 0.5) (layer F.Cu) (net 5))
 (segment (start 83.321 40.903) (end 83.312 40.912) (width 0.5) (layer F.Cu) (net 6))
 (segment (start 85.344 40.903) (end 83.321 40.903) (width 0.5) (layer F.Cu) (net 6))
 (segment (start 83.312 40.912) (end 81.28 40.912) (width 0.5) (layer F.Cu) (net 6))
 (segment (start 81.28 42.559) (end 81.167 42.672) (width 0.5) (layer F.Cu) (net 6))
 (segment (start 81.28 40.912) (end 81.28 42.559) (width 0.5) (layer F.Cu) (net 6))
 (segment (start 81.28 40.337) (end 80.87101 39.92801) (width 0.5) (layer F.Cu) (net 6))
 (segment (start 81.28 40.912) (end 81.28 40.337) (width 0.5) (layer F.Cu) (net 6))
 (segment (start 80.821 39.878) (end 80.87101 39.92801) (width 0.4) (layer F.Cu) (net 6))
 (segment (start 78.8 39.878) (end 80.821 39.878) (width 0.4) (layer F.Cu) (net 6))
 (segment (start 89.154 40.866) (end 89.154 40.894) (width 0.5) (layer F.Cu) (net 9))
 (segment (start 89.154 40.894) (end 87.122 42.926) (width 0.5) (layer F.Cu) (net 9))
 (segment (start 87.122 42.926) (end 87.122 44.704) (width 0.5) (layer F.Cu) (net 9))
 (segment (start 87.122 44.704) (end 86.106 45.72) (width 0.5) (layer F.Cu) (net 9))
 (segment (start 84.083 45.72) (end 83.067 44.704) (width 0.5) (layer F.Cu) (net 9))
 (segment (start 86.106 45.72) (end 84.083 45.72) (width 0.5) (layer F.Cu) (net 9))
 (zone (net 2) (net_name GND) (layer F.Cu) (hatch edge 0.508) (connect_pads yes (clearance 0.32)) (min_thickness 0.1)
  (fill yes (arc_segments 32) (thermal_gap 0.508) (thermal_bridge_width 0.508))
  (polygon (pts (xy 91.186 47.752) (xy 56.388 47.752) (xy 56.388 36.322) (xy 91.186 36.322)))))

